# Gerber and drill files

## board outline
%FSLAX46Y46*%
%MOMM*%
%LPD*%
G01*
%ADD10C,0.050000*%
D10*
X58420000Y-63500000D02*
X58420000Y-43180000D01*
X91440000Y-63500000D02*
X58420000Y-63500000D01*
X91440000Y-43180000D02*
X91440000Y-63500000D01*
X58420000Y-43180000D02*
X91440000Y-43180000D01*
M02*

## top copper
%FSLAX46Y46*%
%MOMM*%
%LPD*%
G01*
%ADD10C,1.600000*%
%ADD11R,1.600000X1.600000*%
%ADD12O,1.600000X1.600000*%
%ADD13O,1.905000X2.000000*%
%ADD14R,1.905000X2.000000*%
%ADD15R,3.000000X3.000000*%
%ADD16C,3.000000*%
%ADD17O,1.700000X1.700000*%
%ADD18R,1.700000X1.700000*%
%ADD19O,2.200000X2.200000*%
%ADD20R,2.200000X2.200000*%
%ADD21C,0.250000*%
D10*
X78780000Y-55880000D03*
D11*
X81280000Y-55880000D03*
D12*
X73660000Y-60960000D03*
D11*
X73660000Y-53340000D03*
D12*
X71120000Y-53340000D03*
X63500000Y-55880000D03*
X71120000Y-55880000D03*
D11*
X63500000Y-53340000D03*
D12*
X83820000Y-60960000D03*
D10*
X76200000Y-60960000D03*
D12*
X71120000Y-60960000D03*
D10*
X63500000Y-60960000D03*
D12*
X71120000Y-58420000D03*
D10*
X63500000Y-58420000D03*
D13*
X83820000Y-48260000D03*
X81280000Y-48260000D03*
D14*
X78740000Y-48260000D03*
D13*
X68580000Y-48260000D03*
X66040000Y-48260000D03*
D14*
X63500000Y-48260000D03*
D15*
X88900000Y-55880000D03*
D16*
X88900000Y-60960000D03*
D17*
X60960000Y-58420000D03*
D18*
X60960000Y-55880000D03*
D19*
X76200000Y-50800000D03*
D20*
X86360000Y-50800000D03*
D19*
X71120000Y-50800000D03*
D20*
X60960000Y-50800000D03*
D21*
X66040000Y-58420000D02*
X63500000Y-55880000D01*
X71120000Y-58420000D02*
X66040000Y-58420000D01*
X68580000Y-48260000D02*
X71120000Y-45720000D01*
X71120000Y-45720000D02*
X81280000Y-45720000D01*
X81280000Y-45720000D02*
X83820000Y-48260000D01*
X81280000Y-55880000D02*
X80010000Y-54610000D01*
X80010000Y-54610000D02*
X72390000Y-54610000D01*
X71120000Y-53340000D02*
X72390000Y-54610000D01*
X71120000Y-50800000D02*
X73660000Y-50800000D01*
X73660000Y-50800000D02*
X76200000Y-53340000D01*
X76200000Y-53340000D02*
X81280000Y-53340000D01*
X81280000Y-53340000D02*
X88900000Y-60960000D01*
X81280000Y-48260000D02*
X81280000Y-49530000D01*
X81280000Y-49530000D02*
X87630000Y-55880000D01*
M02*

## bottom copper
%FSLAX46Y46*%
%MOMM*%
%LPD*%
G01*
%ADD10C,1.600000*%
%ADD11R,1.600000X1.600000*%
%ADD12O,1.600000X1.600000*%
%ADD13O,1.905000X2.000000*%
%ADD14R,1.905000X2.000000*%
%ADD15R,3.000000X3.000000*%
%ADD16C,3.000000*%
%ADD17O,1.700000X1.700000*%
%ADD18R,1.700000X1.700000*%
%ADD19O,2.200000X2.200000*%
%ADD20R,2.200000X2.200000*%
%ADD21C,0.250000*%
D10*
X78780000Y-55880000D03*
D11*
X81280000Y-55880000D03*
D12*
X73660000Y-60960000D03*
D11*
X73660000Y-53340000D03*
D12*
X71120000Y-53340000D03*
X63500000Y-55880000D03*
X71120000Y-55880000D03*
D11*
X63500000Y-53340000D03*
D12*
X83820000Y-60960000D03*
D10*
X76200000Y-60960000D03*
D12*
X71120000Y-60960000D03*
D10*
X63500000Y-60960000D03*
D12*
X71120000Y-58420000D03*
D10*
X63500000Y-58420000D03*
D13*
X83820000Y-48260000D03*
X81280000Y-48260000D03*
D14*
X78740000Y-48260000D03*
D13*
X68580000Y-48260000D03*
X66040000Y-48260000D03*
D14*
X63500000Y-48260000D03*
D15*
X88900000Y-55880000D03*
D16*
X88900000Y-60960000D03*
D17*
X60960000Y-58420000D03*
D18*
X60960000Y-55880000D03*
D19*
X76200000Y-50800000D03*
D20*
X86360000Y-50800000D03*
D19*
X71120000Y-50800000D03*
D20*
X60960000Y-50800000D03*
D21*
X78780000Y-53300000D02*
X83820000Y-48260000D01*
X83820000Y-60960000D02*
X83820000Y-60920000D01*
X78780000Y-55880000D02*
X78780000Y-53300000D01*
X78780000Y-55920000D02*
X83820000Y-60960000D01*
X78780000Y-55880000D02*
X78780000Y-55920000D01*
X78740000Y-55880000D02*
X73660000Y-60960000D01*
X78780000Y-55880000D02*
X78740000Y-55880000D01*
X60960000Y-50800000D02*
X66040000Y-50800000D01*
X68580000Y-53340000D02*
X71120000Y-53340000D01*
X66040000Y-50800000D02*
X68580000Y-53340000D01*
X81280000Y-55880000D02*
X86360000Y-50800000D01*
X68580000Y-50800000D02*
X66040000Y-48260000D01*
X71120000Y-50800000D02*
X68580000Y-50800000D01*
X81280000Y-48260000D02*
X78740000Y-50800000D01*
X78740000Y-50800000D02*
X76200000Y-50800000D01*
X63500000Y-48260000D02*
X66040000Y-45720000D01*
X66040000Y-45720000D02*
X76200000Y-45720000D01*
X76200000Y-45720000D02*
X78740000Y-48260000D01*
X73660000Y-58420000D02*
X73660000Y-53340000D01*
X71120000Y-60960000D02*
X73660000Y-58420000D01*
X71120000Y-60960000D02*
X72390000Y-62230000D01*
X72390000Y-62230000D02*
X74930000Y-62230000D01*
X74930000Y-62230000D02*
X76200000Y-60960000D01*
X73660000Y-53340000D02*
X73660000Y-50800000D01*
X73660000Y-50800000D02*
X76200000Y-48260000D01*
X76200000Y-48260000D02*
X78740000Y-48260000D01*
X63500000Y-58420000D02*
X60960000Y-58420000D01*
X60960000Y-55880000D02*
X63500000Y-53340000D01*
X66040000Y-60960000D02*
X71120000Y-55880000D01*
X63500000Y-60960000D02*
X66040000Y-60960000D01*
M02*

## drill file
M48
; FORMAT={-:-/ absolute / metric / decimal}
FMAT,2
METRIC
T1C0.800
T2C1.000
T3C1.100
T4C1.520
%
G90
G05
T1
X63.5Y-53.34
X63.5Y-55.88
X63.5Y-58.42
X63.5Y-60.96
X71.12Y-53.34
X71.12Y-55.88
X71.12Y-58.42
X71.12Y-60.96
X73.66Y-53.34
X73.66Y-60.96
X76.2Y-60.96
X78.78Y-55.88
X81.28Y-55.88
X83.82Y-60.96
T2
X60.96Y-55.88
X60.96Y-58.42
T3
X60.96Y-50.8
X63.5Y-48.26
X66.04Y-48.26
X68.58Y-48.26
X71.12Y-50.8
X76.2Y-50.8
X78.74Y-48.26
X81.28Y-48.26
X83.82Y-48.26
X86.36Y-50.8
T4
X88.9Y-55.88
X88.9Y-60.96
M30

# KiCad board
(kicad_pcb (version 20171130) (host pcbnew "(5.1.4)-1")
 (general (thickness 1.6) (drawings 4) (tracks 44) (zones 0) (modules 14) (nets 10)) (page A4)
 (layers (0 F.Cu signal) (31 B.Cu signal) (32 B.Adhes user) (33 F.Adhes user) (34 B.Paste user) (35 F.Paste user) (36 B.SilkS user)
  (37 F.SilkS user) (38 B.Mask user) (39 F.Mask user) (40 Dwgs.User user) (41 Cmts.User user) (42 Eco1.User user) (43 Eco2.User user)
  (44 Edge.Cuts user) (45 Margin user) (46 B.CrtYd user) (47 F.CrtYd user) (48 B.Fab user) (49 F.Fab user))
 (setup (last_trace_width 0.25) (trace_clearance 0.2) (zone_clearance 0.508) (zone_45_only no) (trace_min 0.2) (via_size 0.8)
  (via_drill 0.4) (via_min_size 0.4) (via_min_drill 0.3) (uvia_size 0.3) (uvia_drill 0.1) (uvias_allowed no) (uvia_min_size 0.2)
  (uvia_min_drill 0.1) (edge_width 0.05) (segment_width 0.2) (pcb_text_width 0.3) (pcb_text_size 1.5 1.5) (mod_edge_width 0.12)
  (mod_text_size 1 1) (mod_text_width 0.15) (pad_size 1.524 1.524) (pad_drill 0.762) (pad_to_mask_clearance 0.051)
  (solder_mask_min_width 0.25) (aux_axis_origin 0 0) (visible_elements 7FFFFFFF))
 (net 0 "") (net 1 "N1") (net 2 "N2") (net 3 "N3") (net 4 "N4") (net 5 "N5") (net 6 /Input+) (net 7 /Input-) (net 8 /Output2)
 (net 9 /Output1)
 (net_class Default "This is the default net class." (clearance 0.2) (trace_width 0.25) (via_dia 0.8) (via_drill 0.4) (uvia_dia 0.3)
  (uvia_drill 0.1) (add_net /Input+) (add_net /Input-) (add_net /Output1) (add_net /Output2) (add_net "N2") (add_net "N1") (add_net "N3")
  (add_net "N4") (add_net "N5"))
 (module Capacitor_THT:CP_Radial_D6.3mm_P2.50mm (layer F.Cu) (at 81.28 55.88 180)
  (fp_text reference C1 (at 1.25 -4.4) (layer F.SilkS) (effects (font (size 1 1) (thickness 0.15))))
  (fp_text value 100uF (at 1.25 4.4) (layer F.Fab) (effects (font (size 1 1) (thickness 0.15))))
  (pad 2 thru_hole circle (at 2.5 0 180) (size 1.6 1.6) (drill 0.8) (layers *.Cu *.Mask) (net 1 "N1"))
  (pad 1 thru_hole rect (at 0 0 180) (size 1.6 1.6) (drill 0.8) (layers *.Cu *.Mask) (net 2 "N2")))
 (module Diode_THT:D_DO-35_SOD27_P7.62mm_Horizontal (layer F.Cu) (at 73.66 53.34 270)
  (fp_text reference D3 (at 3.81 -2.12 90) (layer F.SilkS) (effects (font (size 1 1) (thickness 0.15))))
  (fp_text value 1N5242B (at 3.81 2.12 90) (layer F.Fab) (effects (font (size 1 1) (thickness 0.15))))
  (pad 2 thru_hole oval (at 7.62 0 270) (size 1.6 1.6) (drill 0.8) (layers *.Cu *.Mask) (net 1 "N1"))
  (pad 1 thru_hole rect (at 0 0 270) (size 1.6 1.6) (drill 0.8) (layers *.Cu *.Mask) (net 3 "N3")))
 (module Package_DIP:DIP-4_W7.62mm (layer F.Cu) (at 63.5 53.34)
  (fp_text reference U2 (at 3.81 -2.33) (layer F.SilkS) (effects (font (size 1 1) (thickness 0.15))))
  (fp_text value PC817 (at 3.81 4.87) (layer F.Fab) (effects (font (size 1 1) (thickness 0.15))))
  (pad 4 thru_hole oval (at 7.62 0) (size 1.6 1.6) (drill 0.8) (layers *.Cu *.Mask) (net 2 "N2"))
  (pad 2 thru_hole oval (at 0 2.54) (size 1.6 1.6) (drill 0.8) (layers *.Cu *.Mask) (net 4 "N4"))
  (pad 3 thru_hole oval (at 7.62 2.54) (size 1.6 1.6) (drill 0.8) (layers *.Cu *.Mask) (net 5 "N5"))
  (pad 1 thru_hole rect (at 0 0) (size 1.6 1.6) (drill 0.8) (layers *.Cu *.Mask) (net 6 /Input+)))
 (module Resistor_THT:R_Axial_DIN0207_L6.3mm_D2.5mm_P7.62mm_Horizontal (layer F.Cu) (at 76.2 60.96)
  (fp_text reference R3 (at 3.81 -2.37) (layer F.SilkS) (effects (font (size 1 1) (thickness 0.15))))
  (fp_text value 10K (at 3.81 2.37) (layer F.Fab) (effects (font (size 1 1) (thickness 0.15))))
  (pad 2 thru_hole oval (at 7.62 0) (size 1.6 1.6) (drill 0.8) (layers *.Cu *.Mask) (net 1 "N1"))
  (pad 1 thru_hole circle (at 0 0) (size 1.6 1.6) (drill 0.8) (layers *.Cu *.Mask) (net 3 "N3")))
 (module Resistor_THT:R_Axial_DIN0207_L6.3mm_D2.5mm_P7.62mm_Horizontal (layer F.Cu) (at 63.5 60.96)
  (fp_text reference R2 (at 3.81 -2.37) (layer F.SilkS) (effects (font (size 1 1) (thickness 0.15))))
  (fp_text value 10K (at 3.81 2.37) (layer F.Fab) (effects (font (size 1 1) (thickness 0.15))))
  (pad 2 thru_hole oval (at 7.62 0) (size 1.6 1.6) (drill 0.8) (layers *.Cu *.Mask) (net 3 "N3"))
  (pad 1 thru_hole circle (at 0 0) (size 1.6 1.6) (drill 0.8) (layers *.Cu *.Mask) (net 5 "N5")))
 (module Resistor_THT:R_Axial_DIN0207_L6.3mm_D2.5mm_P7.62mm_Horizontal (layer F.Cu) (at 63.5 58.42)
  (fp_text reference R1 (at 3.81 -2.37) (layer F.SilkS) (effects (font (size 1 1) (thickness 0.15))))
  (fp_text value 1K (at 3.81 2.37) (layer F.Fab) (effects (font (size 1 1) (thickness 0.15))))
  (pad 2 thru_hole oval (at 7.62 0) (size 1.6 1.6) (drill 0.8) (layers *.Cu *.Mask) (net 4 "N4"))
  (pad 1 thru_hole circle (at 0 0) (size 1.6 1.6) (drill 0.8) (layers *.Cu *.Mask) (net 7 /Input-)))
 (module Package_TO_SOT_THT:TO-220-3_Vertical (layer F.Cu) (at 78.74 48.26)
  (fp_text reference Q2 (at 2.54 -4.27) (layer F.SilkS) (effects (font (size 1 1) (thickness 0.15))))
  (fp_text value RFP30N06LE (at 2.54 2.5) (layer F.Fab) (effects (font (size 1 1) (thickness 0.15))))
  (pad 3 thru_hole oval (at 5.08 0) (size 1.905 2) (drill 1.1) (layers *.Cu *.Mask) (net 1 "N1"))
  (pad 2 thru_hole oval (at 2.54 0) (size 1.905 2) (drill 1.1) (layers *.Cu *.Mask) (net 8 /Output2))
  (pad 1 thru_hole rect (at 0 0) (size 1.905 2) (drill 1.1) (layers *.Cu *.Mask) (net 3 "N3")))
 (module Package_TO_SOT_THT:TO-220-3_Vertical (layer F.Cu) (at 63.5 48.26)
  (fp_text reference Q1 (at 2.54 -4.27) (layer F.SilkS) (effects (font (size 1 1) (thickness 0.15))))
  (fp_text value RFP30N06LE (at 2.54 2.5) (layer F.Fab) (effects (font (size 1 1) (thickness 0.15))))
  (pad 3 thru_hole oval (at 5.08 0) (size 1.905 2) (drill 1.1) (layers *.Cu *.Mask) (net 1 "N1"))
  (pad 2 thru_hole oval (at 2.54 0) (size 1.905 2) (drill 1.1) (layers *.Cu *.Mask) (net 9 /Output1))
  (pad 1 thru_hole rect (at 0 0) (size 1.905 2) (drill 1.1) (layers *.Cu *.Mask) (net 3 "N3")))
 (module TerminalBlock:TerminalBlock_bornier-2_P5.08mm (layer F.Cu) (at 88.9 55.88 270)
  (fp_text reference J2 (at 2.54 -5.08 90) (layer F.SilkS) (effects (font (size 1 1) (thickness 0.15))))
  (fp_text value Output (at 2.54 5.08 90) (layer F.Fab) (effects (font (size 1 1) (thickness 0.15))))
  (pad 1 thru_hole rect (at 0 0 270) (size 3 3) (drill 1.52) (layers *.Cu *.Mask) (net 8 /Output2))
  (pad 2 thru_hole circle (at 5.08 0 270) (size 3 3) (drill 1.52) (layers *.Cu *.Mask) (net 9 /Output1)))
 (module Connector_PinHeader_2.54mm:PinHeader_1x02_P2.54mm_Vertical (layer F.Cu) (at 60.96 55.88)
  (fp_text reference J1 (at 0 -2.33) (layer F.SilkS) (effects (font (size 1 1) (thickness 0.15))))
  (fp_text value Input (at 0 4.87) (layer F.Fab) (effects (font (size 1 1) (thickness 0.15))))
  (pad 2 thru_hole oval (at 0 2.54) (size 1.7 1.7) (drill 1) (layers *.Cu *.Mask) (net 7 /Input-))
  (pad 1 thru_hole rect (at 0 0) (size 1.7 1.7) (drill 1) (layers *.Cu *.Mask) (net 6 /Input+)))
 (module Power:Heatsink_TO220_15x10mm (layer F.Cu) (at 81.28 44.45)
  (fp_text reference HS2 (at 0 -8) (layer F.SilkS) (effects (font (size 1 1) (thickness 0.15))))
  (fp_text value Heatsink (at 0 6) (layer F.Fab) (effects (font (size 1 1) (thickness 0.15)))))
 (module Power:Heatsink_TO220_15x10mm (layer F.Cu) (at 66.04 44.45)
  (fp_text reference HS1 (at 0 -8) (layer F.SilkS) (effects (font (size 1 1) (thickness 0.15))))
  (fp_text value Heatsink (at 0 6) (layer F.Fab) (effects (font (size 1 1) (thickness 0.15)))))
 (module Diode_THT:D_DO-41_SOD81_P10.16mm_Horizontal (layer F.Cu) (at 86.36 50.8 180)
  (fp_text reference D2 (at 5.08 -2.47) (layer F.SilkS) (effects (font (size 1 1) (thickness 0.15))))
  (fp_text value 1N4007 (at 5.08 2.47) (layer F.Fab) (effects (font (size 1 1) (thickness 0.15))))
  (pad 2 thru_hole oval (at 10.16 0 180) (size 2.2 2.2) (drill 1.1) (layers *.Cu *.Mask) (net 8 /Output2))
  (pad 1 thru_hole rect (at 0 0 180) (size 2.2 2.2) (drill 1.1) (layers *.Cu *.Mask) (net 2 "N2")))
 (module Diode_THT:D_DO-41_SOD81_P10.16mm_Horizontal (layer F.Cu) (at 60.96 50.8)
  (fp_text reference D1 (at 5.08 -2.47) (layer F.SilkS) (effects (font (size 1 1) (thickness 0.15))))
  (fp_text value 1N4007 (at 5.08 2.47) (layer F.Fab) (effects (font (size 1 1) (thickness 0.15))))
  (pad 2 thru_hole oval (at 10.16 0) (size 2.2 2.2) (drill 1.1) (layers *.Cu *.Mask) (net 9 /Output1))
  (pad 1 thru_hole rect (at 0 0) (size 2.2 2.2) (drill 1.1) (layers *.Cu *.Mask) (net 2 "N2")))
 (gr_line (start 58.42 63.5) (end 58.42 43.18) (layer Edge.Cuts) (width 0.05))
 (gr_line (start 91.44 63.5) (end 58.42 63.5) (layer Edge.Cuts) (width 0.05))
 (gr_line (start 91.44 43.18) (end 91.44 63.5) (layer Edge.Cuts) (width 0.05))
 (gr_line (start 58.42 43.18) (end 91.44 43.18) (layer Edge.Cuts) (width 0.05))
 (segment (start 66.04 58.42) (end 63.5 55.88) (width 0.25) (layer F.Cu) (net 4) (status 20))
 (segment (start 71.12 58.42) (end 66.04 58.42) (width 0.25) (layer F.Cu) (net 4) (status 10))
 (segment (start 68.58 48.26) (end 71.12 45.72) (width 0.25) (layer F.Cu) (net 1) (status 10))
 (segment (start 71.12 45.72) (end 81.28 45.72) (width 0.25) (layer F.Cu) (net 1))
 (segment (start 81.28 45.72) (end 83.82 48.26) (width 0.25) (layer F.Cu) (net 1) (status 20))
 (segment (start 78.78 53.3) (end 83.82 48.26) (width 0.25) (layer B.Cu) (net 1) (status 20))
 (segment (start 83.82 60.96) (end 83.82 60.92) (width 0.25) (layer B.Cu) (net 1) (status 30))
 (segment (start 78.78 55.88) (end 78.78 53.3) (width 0.25) (layer B.Cu) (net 1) (status 10))
 (segment (start 78.78 55.92) (end 83.82 60.96) (width 0.25) (layer B.Cu) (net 1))
 (segment (start 78.78 55.88) (end 78.78 55.92) (width 0.25) (layer B.Cu) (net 1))
 (segment (start 78.74 55.88) (end 73.66 60.96) (width 0.25) (layer B.Cu) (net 1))
 (segment (start 78.78 55.88) (end 78.74 55.88) (width 0.25) (layer B.Cu) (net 1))
 (segment (start 60.96 50.8) (end 66.04 50.8) (width 0.25) (layer B.Cu) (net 2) (status 10))
 (segment (start 68.58 53.34) (end 71.12 53.34) (width 0.25) (layer B.Cu) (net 2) (status 20))
 (segment (start 66.04 50.8) (end 68.58 53.34) (width 0.25) (layer B.Cu) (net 2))
 (segment (start 81.28 55.88) (end 86.36 50.8) (width 0.25) (layer B.Cu) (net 2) (status 30))
 (segment (start 81.28 55.88) (end 80.01 54.61) (width 0.25) (layer F.Cu) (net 2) (status 10))
 (segment (start 80.01 54.61) (end 72.39 54.61) (width 0.25) (layer F.Cu) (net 2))
 (segment (start 71.12 53.34) (end 72.39 54.61) (width 0.25) (layer F.Cu) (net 2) (status 10))
 (segment (start 68.58 50.8) (end 66.04 48.26) (width 0.25) (layer B.Cu) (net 9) (status 20))
 (segment (start 71.12 50.8) (end 68.58 50.8) (width 0.25) (layer B.Cu) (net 9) (status 10))
 (segment (start 71.12 50.8) (end 73.66 50.8) (width 0.25) (layer F.Cu) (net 9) (status 10))
 (segment (start 73.66 50.8) (end 76.2 53.34) (width 0.25) (layer F.Cu) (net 9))
 (segment (start 76.2 53.34) (end 81.28 53.34) (width 0.25) (layer F.Cu) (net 9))
 (segment (start 81.28 53.34) (end 88.9 60.96) (width 0.25) (layer F.Cu) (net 9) (status 20))
 (segment (start 81.28 48.26) (end 78.74 50.8) (width 0.25) (layer B.Cu) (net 8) (status 10))
 (segment (start 78.74 50.8) (end 76.2 50.8) (width 0.25) (layer B.Cu) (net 8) (status 20))
 (segment (start 81.28 48.26) (end 81.28 49.53) (width 0.25) (layer F.Cu) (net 8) (status 10))
 (segment (start 81.28 49.53) (end 87.63 55.88) (width 0.25) (layer F.Cu) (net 8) (status 20))
 (segment (start 63.5 48.26) (end 66.04 45.72) (width 0.25) (layer B.Cu) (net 3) (status 10))
 (segment (start 66.04 45.72) (end 76.2 45.72) (width 0.25) (layer B.Cu) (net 3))
 (segment (start 76.2 45.72) (end 78.74 48.26) (width 0.25) (layer B.Cu) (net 3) (status 20))
 (segment (start 73.66 58.42) (end 73.66 53.34) (width 0.25) (layer B.Cu) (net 3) (status 20))
 (segment (start 71.12 60.96) (end 73.66 58.42) (width 0.25) (layer B.Cu) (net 3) (status 10))
 (segment (start 71.12 60.96) (end 72.39 62.23) (width 0.25) (layer B.Cu) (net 3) (status 10))
 (segment (start 72.39 62.23) (end 74.93 62.23) (width 0.25) (layer B.Cu) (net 3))
 (segment (start 74.93 62.23) (end 76.2 60.96) (width 0.25) (layer B.Cu) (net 3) (status 20))
 (segment (start 73.66 53.34) (end 73.66 50.8) (width 0.25) (layer B.Cu) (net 3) (status 10))
 (segment (start 73.66 50.8) (end 76.2 48.26) (width 0.25) (layer B.Cu) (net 3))
 (segment (start 76.2 48.26) (end 78.74 48.26) (width 0.25) (layer B.Cu) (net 3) (status 20))
 (segment (start 63.5 58.42) (end 60.96 58.42) (width 0.25) (layer B.Cu) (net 7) (status 30))
 (segment (start 60.96 55.88) (end 63.5 53.34) (width 0.25) (layer B.Cu) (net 6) (status 30))
 (segment (start 66.04 60.96) (end 71.12 55.88) (width 0.25) (layer B.Cu) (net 5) (status 20))
 (segment (start 63.5 60.96) (end 66.04 60.96) (width 0.25) (layer B.Cu) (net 5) (status 10)))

